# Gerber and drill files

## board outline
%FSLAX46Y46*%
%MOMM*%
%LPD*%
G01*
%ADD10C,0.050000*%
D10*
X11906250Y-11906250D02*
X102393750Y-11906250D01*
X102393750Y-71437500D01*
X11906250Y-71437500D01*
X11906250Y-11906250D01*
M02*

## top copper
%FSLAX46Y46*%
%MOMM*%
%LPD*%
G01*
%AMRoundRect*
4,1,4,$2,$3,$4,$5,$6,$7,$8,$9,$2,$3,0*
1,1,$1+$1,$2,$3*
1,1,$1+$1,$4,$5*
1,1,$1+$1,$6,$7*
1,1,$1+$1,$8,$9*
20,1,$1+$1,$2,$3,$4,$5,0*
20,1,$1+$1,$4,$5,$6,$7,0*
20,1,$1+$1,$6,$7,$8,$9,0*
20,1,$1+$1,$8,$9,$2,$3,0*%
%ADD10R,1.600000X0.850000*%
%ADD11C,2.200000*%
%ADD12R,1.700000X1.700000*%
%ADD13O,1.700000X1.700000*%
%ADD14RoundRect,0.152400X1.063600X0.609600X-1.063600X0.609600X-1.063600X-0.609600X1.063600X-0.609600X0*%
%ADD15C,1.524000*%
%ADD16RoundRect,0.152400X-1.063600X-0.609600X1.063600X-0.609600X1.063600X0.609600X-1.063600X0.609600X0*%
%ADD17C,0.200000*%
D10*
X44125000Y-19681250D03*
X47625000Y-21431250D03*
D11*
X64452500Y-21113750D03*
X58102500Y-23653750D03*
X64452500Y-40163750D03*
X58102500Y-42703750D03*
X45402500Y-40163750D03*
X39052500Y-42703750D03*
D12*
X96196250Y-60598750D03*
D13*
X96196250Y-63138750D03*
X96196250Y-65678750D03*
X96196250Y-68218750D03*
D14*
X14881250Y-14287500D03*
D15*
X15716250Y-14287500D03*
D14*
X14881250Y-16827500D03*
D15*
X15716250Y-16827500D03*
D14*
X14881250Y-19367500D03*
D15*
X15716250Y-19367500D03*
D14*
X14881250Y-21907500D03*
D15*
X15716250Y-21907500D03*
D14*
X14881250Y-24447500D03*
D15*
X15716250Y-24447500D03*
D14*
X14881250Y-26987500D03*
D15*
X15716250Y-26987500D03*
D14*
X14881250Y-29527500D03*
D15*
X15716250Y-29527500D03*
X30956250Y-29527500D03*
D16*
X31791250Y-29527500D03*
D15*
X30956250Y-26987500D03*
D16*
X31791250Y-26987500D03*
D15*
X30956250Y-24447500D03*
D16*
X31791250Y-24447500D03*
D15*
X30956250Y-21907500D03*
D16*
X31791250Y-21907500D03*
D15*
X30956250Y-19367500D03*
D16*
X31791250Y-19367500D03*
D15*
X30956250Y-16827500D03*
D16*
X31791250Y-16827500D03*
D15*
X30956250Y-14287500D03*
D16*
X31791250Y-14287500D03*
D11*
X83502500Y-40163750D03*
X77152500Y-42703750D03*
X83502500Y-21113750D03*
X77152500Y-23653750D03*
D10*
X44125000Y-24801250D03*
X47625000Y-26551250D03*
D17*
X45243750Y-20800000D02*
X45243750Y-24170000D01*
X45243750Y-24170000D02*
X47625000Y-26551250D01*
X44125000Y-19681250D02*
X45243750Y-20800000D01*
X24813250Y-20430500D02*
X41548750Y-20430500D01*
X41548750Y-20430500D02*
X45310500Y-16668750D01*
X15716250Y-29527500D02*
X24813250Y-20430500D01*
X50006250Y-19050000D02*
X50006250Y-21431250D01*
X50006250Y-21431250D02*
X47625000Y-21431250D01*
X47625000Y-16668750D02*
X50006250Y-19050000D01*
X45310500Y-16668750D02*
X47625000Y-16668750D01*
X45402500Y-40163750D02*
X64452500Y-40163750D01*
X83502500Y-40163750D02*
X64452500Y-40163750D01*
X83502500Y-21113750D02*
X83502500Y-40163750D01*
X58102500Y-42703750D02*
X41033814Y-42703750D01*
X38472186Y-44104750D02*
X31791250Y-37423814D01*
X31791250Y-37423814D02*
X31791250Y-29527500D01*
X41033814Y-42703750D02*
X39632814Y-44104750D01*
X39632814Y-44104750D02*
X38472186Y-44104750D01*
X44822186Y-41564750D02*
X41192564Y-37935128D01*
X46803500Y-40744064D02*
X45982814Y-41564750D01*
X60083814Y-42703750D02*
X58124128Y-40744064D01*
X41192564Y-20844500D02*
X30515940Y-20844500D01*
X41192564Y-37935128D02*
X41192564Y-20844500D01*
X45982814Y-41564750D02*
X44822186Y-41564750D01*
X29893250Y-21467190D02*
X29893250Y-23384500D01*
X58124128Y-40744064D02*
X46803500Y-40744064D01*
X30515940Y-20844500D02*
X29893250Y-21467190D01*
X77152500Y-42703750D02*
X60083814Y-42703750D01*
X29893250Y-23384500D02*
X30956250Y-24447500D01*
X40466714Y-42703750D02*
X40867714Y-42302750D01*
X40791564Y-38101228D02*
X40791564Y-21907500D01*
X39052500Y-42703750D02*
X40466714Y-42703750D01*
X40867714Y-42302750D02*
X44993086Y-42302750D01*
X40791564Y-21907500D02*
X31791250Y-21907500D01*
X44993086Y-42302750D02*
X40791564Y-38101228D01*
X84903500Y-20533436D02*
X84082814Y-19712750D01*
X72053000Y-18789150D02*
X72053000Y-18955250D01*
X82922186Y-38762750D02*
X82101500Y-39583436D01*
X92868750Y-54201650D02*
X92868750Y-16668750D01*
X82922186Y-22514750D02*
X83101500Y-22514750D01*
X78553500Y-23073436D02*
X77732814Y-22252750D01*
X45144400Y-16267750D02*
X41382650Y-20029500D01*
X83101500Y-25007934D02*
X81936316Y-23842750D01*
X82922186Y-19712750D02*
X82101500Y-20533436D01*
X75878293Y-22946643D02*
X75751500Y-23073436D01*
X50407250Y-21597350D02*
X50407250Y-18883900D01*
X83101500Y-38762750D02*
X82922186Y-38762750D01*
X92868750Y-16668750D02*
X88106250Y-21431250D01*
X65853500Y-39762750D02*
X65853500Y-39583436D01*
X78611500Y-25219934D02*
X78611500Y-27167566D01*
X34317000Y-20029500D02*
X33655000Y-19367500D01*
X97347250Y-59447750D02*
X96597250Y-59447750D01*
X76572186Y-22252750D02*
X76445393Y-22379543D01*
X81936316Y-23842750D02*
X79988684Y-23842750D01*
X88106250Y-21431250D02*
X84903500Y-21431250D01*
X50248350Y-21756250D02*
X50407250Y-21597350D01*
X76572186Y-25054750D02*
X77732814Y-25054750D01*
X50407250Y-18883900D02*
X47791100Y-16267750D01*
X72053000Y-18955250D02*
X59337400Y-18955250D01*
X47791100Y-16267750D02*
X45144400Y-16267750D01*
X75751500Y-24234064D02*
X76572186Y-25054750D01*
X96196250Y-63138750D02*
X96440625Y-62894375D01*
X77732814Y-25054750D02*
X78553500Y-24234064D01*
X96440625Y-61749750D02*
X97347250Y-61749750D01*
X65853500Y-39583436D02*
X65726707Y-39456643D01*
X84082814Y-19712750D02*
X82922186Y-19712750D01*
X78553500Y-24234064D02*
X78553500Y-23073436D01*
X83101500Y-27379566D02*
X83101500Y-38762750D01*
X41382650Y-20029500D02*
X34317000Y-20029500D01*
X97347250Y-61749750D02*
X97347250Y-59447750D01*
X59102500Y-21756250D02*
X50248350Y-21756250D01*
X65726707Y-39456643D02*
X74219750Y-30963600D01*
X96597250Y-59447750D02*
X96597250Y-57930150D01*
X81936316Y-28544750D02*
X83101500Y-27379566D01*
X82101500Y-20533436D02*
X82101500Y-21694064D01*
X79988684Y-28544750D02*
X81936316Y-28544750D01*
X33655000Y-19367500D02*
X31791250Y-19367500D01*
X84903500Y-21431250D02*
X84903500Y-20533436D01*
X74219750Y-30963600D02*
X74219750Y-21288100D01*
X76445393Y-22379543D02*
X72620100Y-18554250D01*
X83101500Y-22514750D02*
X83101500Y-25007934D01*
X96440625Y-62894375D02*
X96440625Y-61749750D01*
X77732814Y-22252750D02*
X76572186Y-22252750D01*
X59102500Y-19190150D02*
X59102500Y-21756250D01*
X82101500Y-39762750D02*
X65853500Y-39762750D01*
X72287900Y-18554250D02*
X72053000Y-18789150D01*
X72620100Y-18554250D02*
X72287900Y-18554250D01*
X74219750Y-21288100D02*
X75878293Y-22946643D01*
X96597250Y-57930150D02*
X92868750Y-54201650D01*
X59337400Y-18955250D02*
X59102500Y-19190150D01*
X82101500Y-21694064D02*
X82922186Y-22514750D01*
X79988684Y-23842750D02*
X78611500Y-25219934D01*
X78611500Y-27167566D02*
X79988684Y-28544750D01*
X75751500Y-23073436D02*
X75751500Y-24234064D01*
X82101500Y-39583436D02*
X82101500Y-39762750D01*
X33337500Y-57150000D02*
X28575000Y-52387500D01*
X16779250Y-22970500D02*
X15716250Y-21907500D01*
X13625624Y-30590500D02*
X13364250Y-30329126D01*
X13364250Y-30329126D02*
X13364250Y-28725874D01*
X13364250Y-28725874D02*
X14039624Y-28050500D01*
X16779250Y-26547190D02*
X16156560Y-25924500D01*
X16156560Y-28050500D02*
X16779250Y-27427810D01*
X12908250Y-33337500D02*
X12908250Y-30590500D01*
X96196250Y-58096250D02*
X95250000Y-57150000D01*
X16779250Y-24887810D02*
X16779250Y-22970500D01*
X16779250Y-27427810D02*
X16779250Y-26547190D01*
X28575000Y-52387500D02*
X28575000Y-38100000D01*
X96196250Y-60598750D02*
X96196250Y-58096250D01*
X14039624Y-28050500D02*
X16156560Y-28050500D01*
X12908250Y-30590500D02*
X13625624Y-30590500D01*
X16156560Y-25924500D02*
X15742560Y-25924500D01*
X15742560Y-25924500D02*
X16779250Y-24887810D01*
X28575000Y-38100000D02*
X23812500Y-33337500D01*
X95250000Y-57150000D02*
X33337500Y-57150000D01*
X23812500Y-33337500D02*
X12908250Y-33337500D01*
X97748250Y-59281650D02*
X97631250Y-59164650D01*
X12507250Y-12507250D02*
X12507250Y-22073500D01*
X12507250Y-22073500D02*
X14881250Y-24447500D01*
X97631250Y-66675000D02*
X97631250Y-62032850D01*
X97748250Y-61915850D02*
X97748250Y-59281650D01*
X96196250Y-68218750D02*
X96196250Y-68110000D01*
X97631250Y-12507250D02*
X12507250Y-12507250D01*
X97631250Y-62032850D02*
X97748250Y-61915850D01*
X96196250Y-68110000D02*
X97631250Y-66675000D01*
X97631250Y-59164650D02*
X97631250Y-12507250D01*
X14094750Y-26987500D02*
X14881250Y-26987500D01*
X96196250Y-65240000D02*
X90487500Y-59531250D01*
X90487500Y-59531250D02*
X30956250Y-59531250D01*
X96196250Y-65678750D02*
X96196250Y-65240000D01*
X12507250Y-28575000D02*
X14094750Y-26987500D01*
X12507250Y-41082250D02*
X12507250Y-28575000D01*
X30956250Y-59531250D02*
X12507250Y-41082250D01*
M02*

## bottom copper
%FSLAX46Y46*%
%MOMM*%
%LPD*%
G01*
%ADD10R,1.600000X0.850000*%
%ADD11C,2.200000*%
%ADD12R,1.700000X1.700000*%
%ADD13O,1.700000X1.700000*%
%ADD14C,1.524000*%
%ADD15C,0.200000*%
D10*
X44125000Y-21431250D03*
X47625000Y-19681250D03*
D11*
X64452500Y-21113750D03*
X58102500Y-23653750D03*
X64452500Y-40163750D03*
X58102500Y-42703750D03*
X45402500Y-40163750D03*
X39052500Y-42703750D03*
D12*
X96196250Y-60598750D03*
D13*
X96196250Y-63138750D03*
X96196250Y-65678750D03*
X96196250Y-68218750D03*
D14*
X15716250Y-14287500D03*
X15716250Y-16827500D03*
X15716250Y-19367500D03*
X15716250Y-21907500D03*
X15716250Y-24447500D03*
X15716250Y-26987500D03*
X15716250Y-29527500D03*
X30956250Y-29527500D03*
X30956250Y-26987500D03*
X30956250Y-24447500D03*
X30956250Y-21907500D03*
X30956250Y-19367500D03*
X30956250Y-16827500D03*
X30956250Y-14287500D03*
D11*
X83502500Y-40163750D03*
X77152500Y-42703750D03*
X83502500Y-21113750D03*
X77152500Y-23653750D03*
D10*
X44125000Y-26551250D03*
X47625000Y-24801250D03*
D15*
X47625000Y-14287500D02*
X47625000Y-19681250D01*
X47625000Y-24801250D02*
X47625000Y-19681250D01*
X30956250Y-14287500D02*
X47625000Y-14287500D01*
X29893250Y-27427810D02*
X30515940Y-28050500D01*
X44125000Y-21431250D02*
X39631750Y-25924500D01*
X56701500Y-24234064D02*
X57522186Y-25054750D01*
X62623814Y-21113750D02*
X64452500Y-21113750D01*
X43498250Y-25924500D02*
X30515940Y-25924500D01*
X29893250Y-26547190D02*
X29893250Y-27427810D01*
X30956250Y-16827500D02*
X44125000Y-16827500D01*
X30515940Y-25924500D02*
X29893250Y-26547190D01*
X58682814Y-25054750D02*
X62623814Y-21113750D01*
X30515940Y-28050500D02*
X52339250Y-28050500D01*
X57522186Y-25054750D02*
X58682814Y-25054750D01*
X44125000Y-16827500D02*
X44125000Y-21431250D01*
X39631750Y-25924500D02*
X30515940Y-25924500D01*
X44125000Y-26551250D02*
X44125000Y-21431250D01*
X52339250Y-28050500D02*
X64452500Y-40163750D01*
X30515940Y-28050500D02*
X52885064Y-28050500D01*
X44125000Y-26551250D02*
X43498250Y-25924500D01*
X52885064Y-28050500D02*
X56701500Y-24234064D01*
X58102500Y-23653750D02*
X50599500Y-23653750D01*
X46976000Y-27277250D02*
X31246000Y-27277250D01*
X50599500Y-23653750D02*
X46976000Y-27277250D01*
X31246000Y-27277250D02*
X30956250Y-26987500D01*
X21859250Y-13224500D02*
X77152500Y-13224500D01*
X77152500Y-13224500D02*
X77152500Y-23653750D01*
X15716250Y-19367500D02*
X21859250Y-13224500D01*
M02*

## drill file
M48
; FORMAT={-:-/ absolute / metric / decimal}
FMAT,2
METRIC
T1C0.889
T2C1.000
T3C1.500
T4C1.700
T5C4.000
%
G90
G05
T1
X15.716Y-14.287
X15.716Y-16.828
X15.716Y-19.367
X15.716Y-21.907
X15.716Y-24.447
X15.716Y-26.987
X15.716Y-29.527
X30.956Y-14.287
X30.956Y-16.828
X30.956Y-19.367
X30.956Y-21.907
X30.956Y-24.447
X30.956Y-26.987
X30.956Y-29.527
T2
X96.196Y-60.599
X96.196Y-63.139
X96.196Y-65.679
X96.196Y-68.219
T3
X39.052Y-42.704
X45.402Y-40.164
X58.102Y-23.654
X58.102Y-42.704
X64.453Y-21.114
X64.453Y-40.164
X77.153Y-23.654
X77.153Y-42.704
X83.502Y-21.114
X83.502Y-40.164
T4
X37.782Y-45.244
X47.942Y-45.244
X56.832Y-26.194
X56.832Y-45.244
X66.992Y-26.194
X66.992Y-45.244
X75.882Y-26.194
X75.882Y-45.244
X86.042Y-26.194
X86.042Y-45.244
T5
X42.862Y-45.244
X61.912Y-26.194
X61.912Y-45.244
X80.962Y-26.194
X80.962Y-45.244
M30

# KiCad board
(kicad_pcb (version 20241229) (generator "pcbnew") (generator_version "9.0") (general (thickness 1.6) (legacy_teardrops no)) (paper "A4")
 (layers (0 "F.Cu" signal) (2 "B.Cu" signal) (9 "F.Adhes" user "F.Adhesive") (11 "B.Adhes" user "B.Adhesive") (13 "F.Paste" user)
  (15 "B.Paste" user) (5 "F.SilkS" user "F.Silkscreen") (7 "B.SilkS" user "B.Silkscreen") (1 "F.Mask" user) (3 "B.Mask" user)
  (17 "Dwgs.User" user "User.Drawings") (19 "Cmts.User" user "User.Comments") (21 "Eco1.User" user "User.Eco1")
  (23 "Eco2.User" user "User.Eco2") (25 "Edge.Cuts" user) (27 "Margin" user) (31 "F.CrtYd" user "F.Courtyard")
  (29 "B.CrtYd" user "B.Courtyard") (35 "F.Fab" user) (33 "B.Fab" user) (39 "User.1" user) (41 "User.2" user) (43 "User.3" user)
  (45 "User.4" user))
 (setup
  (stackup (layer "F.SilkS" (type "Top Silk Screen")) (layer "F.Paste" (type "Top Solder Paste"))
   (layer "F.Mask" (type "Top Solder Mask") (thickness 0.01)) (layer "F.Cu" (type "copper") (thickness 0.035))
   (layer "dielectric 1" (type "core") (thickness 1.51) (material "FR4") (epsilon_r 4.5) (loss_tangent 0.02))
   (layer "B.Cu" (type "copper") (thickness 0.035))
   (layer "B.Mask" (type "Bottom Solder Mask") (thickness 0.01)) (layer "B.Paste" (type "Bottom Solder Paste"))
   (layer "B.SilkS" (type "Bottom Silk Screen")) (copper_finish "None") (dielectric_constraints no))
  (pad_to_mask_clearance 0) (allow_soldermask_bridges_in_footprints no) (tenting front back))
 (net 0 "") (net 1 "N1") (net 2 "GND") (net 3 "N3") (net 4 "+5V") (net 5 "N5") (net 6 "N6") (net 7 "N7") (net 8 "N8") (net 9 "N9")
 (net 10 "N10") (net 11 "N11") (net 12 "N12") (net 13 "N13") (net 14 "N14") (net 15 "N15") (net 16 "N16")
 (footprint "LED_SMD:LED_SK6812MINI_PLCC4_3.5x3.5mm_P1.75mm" (layer "F.Cu") (at 45.875 20.55625)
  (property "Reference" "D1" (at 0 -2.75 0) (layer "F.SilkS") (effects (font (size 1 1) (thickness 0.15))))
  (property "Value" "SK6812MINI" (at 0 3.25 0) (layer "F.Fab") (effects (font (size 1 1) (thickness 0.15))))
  (pad "1" smd rect (at -1.75 -0.875) (size 1.6 0.85) (layers "F.Cu" "F.Mask" "F.Paste") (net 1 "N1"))
  (pad "2" smd rect (at -1.75 0.875) (size 1.6 0.85) (layers "F.Mask" "B.Cu" "F.Paste") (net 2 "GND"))
  (pad "3" smd rect (at 1.75 0.875) (size 1.6 0.85) (layers "F.Cu" "F.Mask" "F.Paste") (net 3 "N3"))
  (pad "4" smd rect (at 1.75 -0.875) (size 1.6 0.85) (layers "F.Mask" "B.Cu" "F.Paste") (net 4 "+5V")))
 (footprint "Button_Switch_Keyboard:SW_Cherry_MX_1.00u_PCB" (layer "F.Cu") (at 64.4525 21.11375)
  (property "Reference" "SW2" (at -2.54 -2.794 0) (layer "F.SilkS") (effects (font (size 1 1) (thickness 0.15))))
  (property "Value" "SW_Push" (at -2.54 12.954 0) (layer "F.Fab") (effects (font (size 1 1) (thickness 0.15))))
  (pad "" np_thru_hole circle (at -7.62 5.08) (size 1.7 1.7) (drill 1.7) (layers "*.Cu" "*.Mask"))
  (pad "" np_thru_hole circle (at -2.54 5.08) (size 4 4) (drill 4) (layers "*.Cu" "*.Mask"))
  (pad "" np_thru_hole circle (at 2.54 5.08) (size 1.7 1.7) (drill 1.7) (layers "*.Cu" "*.Mask"))
  (pad "1" thru_hole circle (at 0 0) (size 2.2 2.2) (drill 1.5) (layers "*.Cu" "*.Mask") (remove_unused_layers no) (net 2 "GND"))
  (pad "2" thru_hole circle (at -6.35 2.54) (size 2.2 2.2) (drill 1.5) (layers "*.Cu" "*.Mask") (remove_unused_layers no) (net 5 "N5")))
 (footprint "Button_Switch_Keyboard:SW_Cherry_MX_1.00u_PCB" (layer "F.Cu") (at 64.4525 40.16375)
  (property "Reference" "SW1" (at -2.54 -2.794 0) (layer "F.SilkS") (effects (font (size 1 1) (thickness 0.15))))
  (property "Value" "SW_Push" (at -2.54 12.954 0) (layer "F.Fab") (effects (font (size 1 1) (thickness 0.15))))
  (pad "" np_thru_hole circle (at -7.62 5.08) (size 1.7 1.7) (drill 1.7) (layers "*.Cu" "*.Mask"))
  (pad "" np_thru_hole circle (at -2.54 5.08) (size 4 4) (drill 4) (layers "*.Cu" "*.Mask"))
  (pad "" np_thru_hole circle (at 2.54 5.08) (size 1.7 1.7) (drill 1.7) (layers "*.Cu" "*.Mask"))
  (pad "1" thru_hole circle (at 0 0) (size 2.2 2.2) (drill 1.5) (layers "*.Cu" "*.Mask") (remove_unused_layers no) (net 2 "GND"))
  (pad "2" thru_hole circle (at -6.35 2.54) (size 2.2 2.2) (drill 1.5) (layers "*.Cu" "*.Mask") (remove_unused_layers no) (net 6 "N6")))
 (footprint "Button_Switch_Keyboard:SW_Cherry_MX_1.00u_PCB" (layer "F.Cu") (at 45.4025 40.16375)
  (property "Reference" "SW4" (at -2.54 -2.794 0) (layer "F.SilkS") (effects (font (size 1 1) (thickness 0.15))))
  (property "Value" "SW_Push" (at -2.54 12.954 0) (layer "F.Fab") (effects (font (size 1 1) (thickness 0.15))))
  (pad "" np_thru_hole circle (at -7.62 5.08) (size 1.7 1.7) (drill 1.7) (layers "*.Cu" "*.Mask"))
  (pad "" np_thru_hole circle (at -2.54 5.08) (size 4 4) (drill 4) (layers "*.Cu" "*.Mask"))
  (pad "" np_thru_hole circle (at 2.54 5.08) (size 1.7 1.7) (drill 1.7) (layers "*.Cu" "*.Mask"))
  (pad "1" thru_hole circle (at 0 0) (size 2.2 2.2) (drill 1.5) (layers "*.Cu" "*.Mask") (remove_unused_layers no) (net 2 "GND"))
  (pad "2" thru_hole circle (at -6.35 2.54) (size 2.2 2.2) (drill 1.5) (layers "*.Cu" "*.Mask") (remove_unused_layers no) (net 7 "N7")))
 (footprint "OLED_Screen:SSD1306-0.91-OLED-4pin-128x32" (layer "F.Cu") (at 59.69625 58.40875)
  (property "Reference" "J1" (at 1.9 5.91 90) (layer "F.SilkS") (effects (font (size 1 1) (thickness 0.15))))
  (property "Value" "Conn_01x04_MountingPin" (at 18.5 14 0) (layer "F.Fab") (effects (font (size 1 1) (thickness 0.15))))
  (pad "1" thru_hole rect (at 36.5 2.19) (size 1.7 1.7) (drill 1) (layers "*.Cu" "*.Mask") (remove_unused_layers no) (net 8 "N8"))
  (pad "2" thru_hole oval (at 36.5 4.73) (size 1.7 1.7) (drill 1) (layers "*.Cu" "*.Mask") (remove_unused_layers no) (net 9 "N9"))
  (pad "3" thru_hole oval (at 36.5 7.27) (size 1.7 1.7) (drill 1) (layers "*.Cu" "*.Mask") (remove_unused_layers no) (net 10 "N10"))
  (pad "4" thru_hole oval (at 36.5 9.81) (size 1.7 1.7) (drill 1) (layers "*.Cu" "*.Mask") (remove_unused_layers no) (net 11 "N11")))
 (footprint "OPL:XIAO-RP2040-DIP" (layer "F.Cu") (at 23.33625 21.9075)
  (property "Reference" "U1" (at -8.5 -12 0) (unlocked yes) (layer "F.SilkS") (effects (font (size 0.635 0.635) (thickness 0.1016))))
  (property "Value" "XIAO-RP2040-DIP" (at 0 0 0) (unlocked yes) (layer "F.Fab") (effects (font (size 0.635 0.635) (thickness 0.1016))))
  (pad "1" smd roundrect (at -8.455 -7.62 180) (size 2.432 1.524) (layers "F.Cu" "F.Mask") (roundrect_rratio 0.1) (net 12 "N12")
   (thermal_bridge_angle 45))
  (pad "1" thru_hole circle (at -7.62 -7.62 180) (size 1.524 1.524) (drill 0.889) (layers "*.Cu" "*.Mask") (remove_unused_layers no)
   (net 12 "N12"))
  (pad "2" smd roundrect (at -8.455 -5.08 180) (size 2.432 1.524) (layers "F.Cu" "F.Mask") (roundrect_rratio 0.1) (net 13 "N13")
   (thermal_bridge_angle 45))
  (pad "2" thru_hole circle (at -7.62 -5.08 180) (size 1.524 1.524) (drill 0.889) (layers "*.Cu" "*.Mask") (remove_unused_layers no)
   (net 13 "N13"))
  (pad "3" smd roundrect (at -8.455 -2.54 180) (size 2.432 1.524) (layers "F.Cu" "F.Mask") (roundrect_rratio 0.1) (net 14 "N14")
   (thermal_bridge_angle 45))
  (pad "3" thru_hole circle (at -7.62 -2.54 180) (size 1.524 1.524) (drill 0.889) (layers "*.Cu" "*.Mask") (remove_unused_layers no)
   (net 14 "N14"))
  (pad "4" smd roundrect (at -8.455 0 180) (size 2.432 1.524) (layers "F.Cu" "F.Mask") (roundrect_rratio 0.1) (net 8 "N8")
   (thermal_bridge_angle 45))
  (pad "4" thru_hole circle (at -7.62 0 180) (size 1.524 1.524) (drill 0.889) (layers "*.Cu" "*.Mask") (remove_unused_layers no)
   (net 8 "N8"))
  (pad "5" smd roundrect (at -8.455 2.54 180) (size 2.432 1.524) (layers "F.Cu" "F.Mask") (roundrect_rratio 0.1) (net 11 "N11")
   (thermal_bridge_angle 45))
  (pad "5" thru_hole circle (at -7.62 2.54 180) (size 1.524 1.524) (drill 0.889) (layers "*.Cu" "*.Mask") (remove_unused_layers no)
   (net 11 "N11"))
  (pad "6" smd roundrect (at -8.455 5.08 180) (size 2.432 1.524) (layers "F.Cu" "F.Mask") (roundrect_rratio 0.1) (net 10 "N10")
   (thermal_bridge_angle 45))
  (pad "6" thru_hole circle (at -7.62 5.08 180) (size 1.524 1.524) (drill 0.889) (layers "*.Cu" "*.Mask") (remove_unused_layers no)
   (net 10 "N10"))
  (pad "7" smd roundrect (at -8.455 7.62 180) (size 2.432 1.524) (layers "F.Cu" "F.Mask") (roundrect_rratio 0.1) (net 3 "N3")
   (thermal_bridge_angle 45))
  (pad "7" thru_hole circle (at -7.62 7.62 180) (size 1.524 1.524) (drill 0.889) (layers "*.Cu" "*.Mask") (remove_unused_layers no)
   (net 3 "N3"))
  (pad "8" thru_hole circle (at 7.62 7.62) (size 1.524 1.524) (drill 0.889) (layers "*.Cu" "*.Mask") (remove_unused_layers no) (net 6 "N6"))
  (pad "8" smd roundrect (at 8.455 7.62) (size 2.432 1.524) (layers "F.Cu" "F.Mask") (roundrect_rratio 0.1) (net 6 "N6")
   (thermal_bridge_angle 45))
  (pad "9" thru_hole circle (at 7.62 5.08) (size 1.524 1.524) (drill 0.889) (layers "*.Cu" "*.Mask") (remove_unused_layers no) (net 5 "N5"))
  (pad "9" smd roundrect (at 8.455 5.08) (size 2.432 1.524) (layers "F.Cu" "F.Mask") (roundrect_rratio 0.1) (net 5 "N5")
   (thermal_bridge_angle 45))
  (pad "10" thru_hole circle (at 7.62 2.54) (size 1.524 1.524) (drill 0.889) (layers "*.Cu" "*.Mask") (remove_unused_layers no)
   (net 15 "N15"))
  (pad "10" smd roundrect (at 8.455 2.54) (size 2.432 1.524) (layers "F.Cu" "F.Mask") (roundrect_rratio 0.1) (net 15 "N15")
   (thermal_bridge_angle 45))
  (pad "11" thru_hole circle (at 7.62 0) (size 1.524 1.524) (drill 0.889) (layers "*.Cu" "*.Mask") (remove_unused_layers no) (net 7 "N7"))
  (pad "11" smd roundrect (at 8.455 0) (size 2.432 1.524) (layers "F.Cu" "F.Mask") (roundrect_rratio 0.1) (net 7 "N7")
   (thermal_bridge_angle 45))
  (pad "12" thru_hole circle (at 7.62 -2.54) (size 1.524 1.524) (drill 0.889) (layers "*.Cu" "*.Mask") (remove_unused_layers no)
   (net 9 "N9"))
  (pad "12" smd roundrect (at 8.455 -2.54) (size 2.432 1.524) (layers "F.Cu" "F.Mask") (roundrect_rratio 0.1) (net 9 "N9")
   (thermal_bridge_angle 45))
  (pad "13" thru_hole circle (at 7.62 -5.08) (size 1.524 1.524) (drill 0.889) (layers "*.Cu" "*.Mask") (remove_unused_layers no)
   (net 2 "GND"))
  (pad "13" smd roundrect (at 8.455 -5.08) (size 2.432 1.524) (layers "F.Cu" "F.Mask") (roundrect_rratio 0.1) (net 2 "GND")
   (thermal_bridge_angle 45))
  (pad "14" thru_hole circle (at 7.62 -7.62) (size 1.524 1.524) (drill 0.889) (layers "*.Cu" "*.Mask") (remove_unused_layers no)
   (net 4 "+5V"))
  (pad "14" smd roundrect (at 8.455 -7.62) (size 2.432 1.524) (layers "F.Cu" "F.Mask") (roundrect_rratio 0.1) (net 4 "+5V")
   (thermal_bridge_angle 45)))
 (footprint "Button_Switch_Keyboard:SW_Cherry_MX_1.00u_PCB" (layer "F.Cu") (at 83.5025 40.16375)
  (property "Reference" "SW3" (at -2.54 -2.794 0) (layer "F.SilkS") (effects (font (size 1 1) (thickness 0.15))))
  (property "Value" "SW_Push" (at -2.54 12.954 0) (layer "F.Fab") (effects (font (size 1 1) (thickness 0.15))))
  (pad "" np_thru_hole circle (at -7.62 5.08) (size 1.7 1.7) (drill 1.7) (layers "*.Cu" "*.Mask"))
  (pad "" np_thru_hole circle (at -2.54 5.08) (size 4 4) (drill 4) (layers "*.Cu" "*.Mask"))
  (pad "" np_thru_hole circle (at 2.54 5.08) (size 1.7 1.7) (drill 1.7) (layers "*.Cu" "*.Mask"))
  (pad "1" thru_hole circle (at 0 0) (size 2.2 2.2) (drill 1.5) (layers "*.Cu" "*.Mask") (remove_unused_layers no) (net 2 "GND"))
  (pad "2" thru_hole circle (at -6.35 2.54) (size 2.2 2.2) (drill 1.5) (layers "*.Cu" "*.Mask") (remove_unused_layers no) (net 15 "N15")))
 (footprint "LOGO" (layer "F.Cu") (at 21.43125 61.9125)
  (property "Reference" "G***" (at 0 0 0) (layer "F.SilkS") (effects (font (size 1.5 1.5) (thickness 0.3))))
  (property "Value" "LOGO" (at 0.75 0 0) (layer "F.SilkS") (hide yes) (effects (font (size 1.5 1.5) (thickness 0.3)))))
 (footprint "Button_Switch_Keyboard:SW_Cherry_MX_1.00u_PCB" (layer "F.Cu") (at 83.5025 21.11375)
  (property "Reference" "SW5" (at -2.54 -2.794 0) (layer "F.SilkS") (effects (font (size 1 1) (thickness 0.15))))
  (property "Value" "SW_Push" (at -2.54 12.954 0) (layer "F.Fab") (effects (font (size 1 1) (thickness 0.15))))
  (pad "" np_thru_hole circle (at -7.62 5.08) (size 1.7 1.7) (drill 1.7) (layers "*.Cu" "*.Mask"))
  (pad "" np_thru_hole circle (at -2.54 5.08) (size 4 4) (drill 4) (layers "*.Cu" "*.Mask"))
  (pad "" np_thru_hole circle (at 2.54 5.08) (size 1.7 1.7) (drill 1.7) (layers "*.Cu" "*.Mask"))
  (pad "1" thru_hole circle (at 0 0) (size 2.2 2.2) (drill 1.5) (layers "*.Cu" "*.Mask") (remove_unused_layers no) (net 2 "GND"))
  (pad "2" thru_hole circle (at -6.35 2.54) (size 2.2 2.2) (drill 1.5) (layers "*.Cu" "*.Mask") (remove_unused_layers no) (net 14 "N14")))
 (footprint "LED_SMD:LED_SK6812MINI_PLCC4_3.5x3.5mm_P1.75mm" (layer "F.Cu") (at 45.875 25.67625)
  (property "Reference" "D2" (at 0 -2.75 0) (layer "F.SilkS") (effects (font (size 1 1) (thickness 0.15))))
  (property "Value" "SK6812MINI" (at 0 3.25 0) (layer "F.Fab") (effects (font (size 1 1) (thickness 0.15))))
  (pad "1" smd rect (at -1.75 -0.875) (size 1.6 0.85) (layers "F.Cu" "F.Mask" "F.Paste") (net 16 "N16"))
  (pad "2" smd rect (at -1.75 0.875) (size 1.6 0.85) (layers "F.Mask" "B.Cu" "F.Paste") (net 2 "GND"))
  (pad "3" smd rect (at 1.75 0.875) (size 1.6 0.85) (layers "F.Cu" "F.Mask" "F.Paste") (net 1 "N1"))
  (pad "4" smd rect (at 1.75 -0.875) (size 1.6 0.85) (layers "F.Mask" "B.Cu" "F.Paste") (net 4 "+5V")))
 (gr_rect (start 11.90625 11.90625) (end 102.39375 71.4375) (stroke (width 0.05) (type default)) (fill no) (layer "Edge.Cuts"))
 (segment (start 45.24375 20.8) (end 45.24375 24.17) (width 0.2) (layer "F.Cu") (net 1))
 (segment (start 45.24375 24.17) (end 47.625 26.55125) (width 0.2) (layer "F.Cu") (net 1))
 (segment (start 44.125 19.68125) (end 45.24375 20.8) (width 0.2) (layer "F.Cu") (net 1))
 (segment (start 47.625 14.2875) (end 47.625 19.68125) (width 0.2) (layer "B.Cu") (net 4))
 (segment (start 47.625 24.80125) (end 47.625 19.68125) (width 0.2) (layer "B.Cu") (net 4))
 (segment (start 30.95625 14.2875) (end 47.625 14.2875) (width 0.2) (layer "B.Cu") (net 4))
 (segment (start 24.81325 20.4305) (end 41.54875 20.4305) (width 0.2) (layer "F.Cu") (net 3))
 (segment (start 41.54875 20.4305) (end 45.3105 16.66875) (width 0.2) (layer "F.Cu") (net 3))
 (segment (start 15.71625 29.5275) (end 24.81325 20.4305) (width 0.2) (layer "F.Cu") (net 3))
 (segment (start 50.00625 19.05) (end 50.00625 21.43125) (width 0.2) (layer "F.Cu") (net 3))
 (segment (start 50.00625 21.43125) (end 47.625 21.43125) (width 0.2) (layer "F.Cu") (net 3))
 (segment (start 47.625 16.66875) (end 50.00625 19.05) (width 0.2) (layer "F.Cu") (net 3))
 (segment (start 45.3105 16.66875) (end 47.625 16.66875) (width 0.2) (layer "F.Cu") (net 3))
 (segment (start 45.4025 40.16375) (end 64.4525 40.16375) (width 0.2) (layer "F.Cu") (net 2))
 (segment (start 83.5025 40.16375) (end 64.4525 40.16375) (width 0.2) (layer "F.Cu") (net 2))
 (segment (start 83.5025 21.11375) (end 83.5025 40.16375) (width 0.2) (layer "F.Cu") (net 2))
 (segment (start 29.89325 27.42781) (end 30.51594 28.0505) (width 0.2) (layer "B.Cu") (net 2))
 (segment (start 44.125 21.43125) (end 39.63175 25.9245) (width 0.2) (layer "B.Cu") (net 2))
 (segment (start 56.7015 24.234064) (end 57.522186 25.05475) (width 0.2) (layer "B.Cu") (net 2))
 (segment (start 62.623814 21.11375) (end 64.4525 21.11375) (width 0.2) (layer "B.Cu") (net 2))
 (segment (start 43.49825 25.9245) (end 30.51594 25.9245) (width 0.2) (layer "B.Cu") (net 2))
 (segment (start 29.89325 26.54719) (end 29.89325 27.42781) (width 0.2) (layer "B.Cu") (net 2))
 (segment (start 30.95625 16.8275) (end 44.125 16.8275) (width 0.2) (layer "B.Cu") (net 2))
 (segment (start 30.51594 25.9245) (end 29.89325 26.54719) (width 0.2) (layer "B.Cu") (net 2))
 (segment (start 58.682814 25.05475) (end 62.623814 21.11375) (width 0.2) (layer "B.Cu") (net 2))
 (segment (start 30.51594 28.0505) (end 52.33925 28.0505) (width 0.2) (layer "B.Cu") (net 2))
 (segment (start 57.522186 25.05475) (end 58.682814 25.05475) (width 0.2) (layer "B.Cu") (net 2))
 (segment (start 44.125 16.8275) (end 44.125 21.43125) (width 0.2) (layer "B.Cu") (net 2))
 (segment (start 39.63175 25.9245) (end 30.51594 25.9245) (width 0.2) (layer "B.Cu") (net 2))
 (segment (start 44.125 26.55125) (end 44.125 21.43125) (width 0.2) (layer "B.Cu") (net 2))
 (segment (start 52.33925 28.0505) (end 64.4525 40.16375) (width 0.2) (layer "B.Cu") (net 2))
 (segment (start 30.51594 28.0505) (end 52.885064 28.0505) (width 0.2) (layer "B.Cu") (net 2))
 (segment (start 44.125 26.55125) (end 43.49825 25.9245) (width 0.2) (layer "B.Cu") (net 2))
 (segment (start 52.885064 28.0505) (end 56.7015 24.234064) (width 0.2) (layer "B.Cu") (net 2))
 (segment (start 58.1025 42.70375) (end 41.033814 42.70375) (width 0.2) (layer "F.Cu") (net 6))
 (segment (start 38.472186 44.10475) (end 31.79125 37.423814) (width 0.2) (layer "F.Cu") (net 6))
 (segment (start 31.79125 37.423814) (end 31.79125 29.5275) (width 0.2) (layer "F.Cu") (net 6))
 (segment (start 41.033814 42.70375) (end 39.632814 44.10475) (width 0.2) (layer "F.Cu") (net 6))
 (segment (start 39.632814 44.10475) (end 38.472186 44.10475) (width 0.2) (layer "F.Cu") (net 6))
 (segment (start 58.1025 23.65375) (end 50.5995 23.65375) (width 0.2) (layer "B.Cu") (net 5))
 (segment (start 46.976 27.27725) (end 31.246 27.27725) (width 0.2) (layer "B.Cu") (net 5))
 (segment (start 50.5995 23.65375) (end 46.976 27.27725) (width 0.2) (layer "B.Cu") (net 5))
 (segment (start 31.246 27.27725) (end 30.95625 26.9875) (width 0.2) (layer "B.Cu") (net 5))
 (segment (start 44.822186 41.56475) (end 41.192564 37.935128) (width 0.2) (layer "F.Cu") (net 15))
 (segment (start 46.8035 40.744064) (end 45.982814 41.56475) (width 0.2) (layer "F.Cu") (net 15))
 (segment (start 60.083814 42.70375) (end 58.124128 40.744064) (width 0.2) (layer "F.Cu") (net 15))
 (segment (start 41.192564 20.8445) (end 30.51594 20.8445) (width 0.2) (layer "F.Cu") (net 15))
 (segment (start 41.192564 37.935128) (end 41.192564 20.8445) (width 0.2) (layer "F.Cu") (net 15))
 (segment (start 45.982814 41.56475) (end 44.822186 41.56475) (width 0.2) (layer "F.Cu") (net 15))
 (segment (start 29.89325 21.46719) (end 29.89325 23.3845) (width 0.2) (layer "F.Cu") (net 15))
 (segment (start 58.124128 40.744064) (end 46.8035 40.744064) (width 0.2) (layer "F.Cu") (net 15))
 (segment (start 30.51594 20.8445) (end 29.89325 21.46719) (width 0.2) (layer "F.Cu") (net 15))
 (segment (start 77.1525 42.70375) (end 60.083814 42.70375) (width 0.2) (layer "F.Cu") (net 15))
 (segment (start 29.89325 23.3845) (end 30.95625 24.4475) (width 0.2) (layer "F.Cu") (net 15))
 (segment (start 40.466714 42.70375) (end 40.867714 42.30275) (width 0.2) (layer "F.Cu") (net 7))
 (segment (start 40.791564 38.101228) (end 40.791564 21.9075) (width 0.2) (layer "F.Cu") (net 7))
 (segment (start 39.0525 42.70375) (end 40.466714 42.70375) (width 0.2) (layer "F.Cu") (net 7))
 (segment (start 40.867714 42.30275) (end 44.993086 42.30275) (width 0.2) (layer "F.Cu") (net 7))
 (segment (start 40.791564 21.9075) (end 31.79125 21.9075) (width 0.2) (layer "F.Cu") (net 7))
 (segment (start 44.993086 42.30275) (end 40.791564 38.101228) (width 0.2) (layer "F.Cu") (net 7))
 (segment (start 84.9035 20.533436) (end 84.082814 19.71275) (width 0.2) (layer "F.Cu") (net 9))
 (segment (start 72.053 18.78915) (end 72.053 18.95525) (width 0.2) (layer "F.Cu") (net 9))
 (segment (start 82.922186 38.76275) (end 82.1015 39.583436) (width 0.2) (layer "F.Cu") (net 9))
 (segment (start 92.86875 54.20165) (end 92.86875 16.66875) (width 0.2) (layer "F.Cu") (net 9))
 (segment (start 82.922186 22.51475) (end 83.1015 22.51475) (width 0.2) (layer "F.Cu") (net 9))
 (segment (start 78.5535 23.073436) (end 77.732814 22.25275) (width 0.2) (layer "F.Cu") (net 9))
 (segment (start 45.1444 16.26775) (end 41.38265 20.0295) (width 0.2) (layer "F.Cu") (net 9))
 (segment (start 83.1015 25.007934) (end 81.936316 23.84275) (width 0.2) (layer "F.Cu") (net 9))
 (segment (start 82.922186 19.71275) (end 82.1015 20.533436) (width 0.2) (layer "F.Cu") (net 9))
 (segment (start 75.878293 22.946643) (end 75.7515 23.073436) (width 0.2) (layer "F.Cu") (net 9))
 (segment (start 50.40725 21.59735) (end 50.40725 18.8839) (width 0.2) (layer "F.Cu") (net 9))
 (segment (start 83.1015 38.76275) (end 82.922186 38.76275) (width 0.2) (layer "F.Cu") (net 9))
 (segment (start 92.86875 16.66875) (end 88.10625 21.43125) (width 0.2) (layer "F.Cu") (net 9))
 (segment (start 65.8535 39.76275) (end 65.8535 39.583436) (width 0.2) (layer "F.Cu") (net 9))
 (segment (start 78.6115 25.219934) (end 78.6115 27.167566) (width 0.2) (layer "F.Cu") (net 9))
 (segment (start 34.317 20.0295) (end 33.655 19.3675) (width 0.2) (layer "F.Cu") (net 9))
 (segment (start 97.34725 59.44775) (end 96.59725 59.44775) (width 0.2) (layer "F.Cu") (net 9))
 (segment (start 76.572186 22.25275) (end 76.445393 22.379543) (width 0.2) (layer "F.Cu") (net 9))
 (segment (start 81.936316 23.84275) (end 79.988684 23.84275) (width 0.2) (layer "F.Cu") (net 9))
 (segment (start 88.10625 21.43125) (end 84.9035 21.43125) (width 0.2) (layer "F.Cu") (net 9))
 (segment (start 50.24835 21.75625) (end 50.40725 21.59735) (width 0.2) (layer "F.Cu") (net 9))
 (segment (start 76.572186 25.05475) (end 77.732814 25.05475) (width 0.2) (layer "F.Cu") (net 9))
 (segment (start 50.40725 18.8839) (end 47.7911 16.26775) (width 0.2) (layer "F.Cu") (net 9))
 (segment (start 72.053 18.95525) (end 59.3374 18.95525) (width 0.2) (layer "F.Cu") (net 9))
 (segment (start 47.7911 16.26775) (end 45.1444 16.26775) (width 0.2) (layer "F.Cu") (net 9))
 (segment (start 75.7515 24.234064) (end 76.572186 25.05475) (width 0.2) (layer "F.Cu") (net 9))
 (segment (start 96.19625 63.13875) (end 96.440625 62.894375) (width 0.2) (layer "F.Cu") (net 9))
 (segment (start 77.732814 25.05475) (end 78.5535 24.234064) (width 0.2) (layer "F.Cu") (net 9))
 (segment (start 96.440625 61.74975) (end 97.34725 61.74975) (width 0.2) (layer "F.Cu") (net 9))
 (segment (start 65.8535 39.583436) (end 65.726707 39.456643) (width 0.2) (layer "F.Cu") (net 9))
 (segment (start 84.082814 19.71275) (end 82.922186 19.71275) (width 0.2) (layer "F.Cu") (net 9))
 (segment (start 78.5535 24.234064) (end 78.5535 23.073436) (width 0.2) (layer "F.Cu") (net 9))
 (segment (start 83.1015 27.379566) (end 83.1015 38.76275) (width 0.2) (layer "F.Cu") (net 9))
 (segment (start 41.38265 20.0295) (end 34.317 20.0295) (width 0.2) (layer "F.Cu") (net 9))
 (segment (start 97.34725 61.74975) (end 97.34725 59.44775) (width 0.2) (layer "F.Cu") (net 9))
 (segment (start 59.1025 21.75625) (end 50.24835 21.75625) (width 0.2) (layer "F.Cu") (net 9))
 (segment (start 65.726707 39.456643) (end 74.21975 30.9636) (width 0.2) (layer "F.Cu") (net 9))
 (segment (start 96.59725 59.44775) (end 96.59725 57.93015) (width 0.2) (layer "F.Cu") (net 9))
 (segment (start 81.936316 28.54475) (end 83.1015 27.379566) (width 0.2) (layer "F.Cu") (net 9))
 (segment (start 82.1015 20.533436) (end 82.1015 21.694064) (width 0.2) (layer "F.Cu") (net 9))
 (segment (start 79.988684 28.54475) (end 81.936316 28.54475) (width 0.2) (layer "F.Cu") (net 9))
 (segment (start 33.655 19.3675) (end 31.79125 19.3675) (width 0.2) (layer "F.Cu") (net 9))
 (segment (start 84.9035 21.43125) (end 84.9035 20.533436) (width 0.2) (layer "F.Cu") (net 9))
 (segment (start 74.21975 30.9636) (end 74.21975 21.2881) (width 0.2) (layer "F.Cu") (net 9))
 (segment (start 76.445393 22.379543) (end 72.6201 18.55425) (width 0.2) (layer "F.Cu") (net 9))
 (segment (start 83.1015 22.51475) (end 83.1015 25.007934) (width 0.2) (layer "F.Cu") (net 9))
 (segment (start 96.440625 62.894375) (end 96.440625 61.74975) (width 0.2) (layer "F.Cu") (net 9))
 (segment (start 77.732814 22.25275) (end 76.572186 22.25275) (width 0.2) (layer "F.Cu") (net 9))
 (segment (start 59.1025 19.19015) (end 59.1025 21.75625) (width 0.2) (layer "F.Cu") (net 9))
 (segment (start 82.1015 39.76275) (end 65.8535 39.76275) (width 0.2) (layer "F.Cu") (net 9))
 (segment (start 72.2879 18.55425) (end 72.053 18.78915) (width 0.2) (layer "F.Cu") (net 9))
 (segment (start 72.6201 18.55425) (end 72.2879 18.55425) (width 0.2) (layer "F.Cu") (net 9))
 (segment (start 74.21975 21.2881) (end 75.878293 22.946643) (width 0.2) (layer "F.Cu") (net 9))
 (segment (start 96.59725 57.93015) (end 92.86875 54.20165) (width 0.2) (layer "F.Cu") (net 9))
 (segment (start 59.3374 18.95525) (end 59.1025 19.19015) (width 0.2) (layer "F.Cu") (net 9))
 (segment (start 82.1015 21.694064) (end 82.922186 22.51475) (width 0.2) (layer "F.Cu") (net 9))
 (segment (start 79.988684 23.84275) (end 78.6115 25.219934) (width 0.2) (layer "F.Cu") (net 9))
 (segment (start 78.6115 27.167566) (end 79.988684 28.54475) (width 0.2) (layer "F.Cu") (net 9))
 (segment (start 75.7515 23.073436) (end 75.7515 24.234064) (width 0.2) (layer "F.Cu") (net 9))
 (segment (start 82.1015 39.583436) (end 82.1015 39.76275) (width 0.2) (layer "F.Cu") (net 9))
 (segment (start 33.3375 57.15) (end 28.575 52.3875) (width 0.2) (layer "F.Cu") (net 8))
 (segment (start 16.77925 22.9705) (end 15.71625 21.9075) (width 0.2) (layer "F.Cu") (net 8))
 (segment (start 13.625624 30.5905) (end 13.36425 30.329126) (width 0.2) (layer "F.Cu") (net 8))
 (segment (start 13.36425 30.329126) (end 13.36425 28.725874) (width 0.2) (layer "F.Cu") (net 8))
 (segment (start 13.36425 28.725874) (end 14.039624 28.0505) (width 0.2) (layer "F.Cu") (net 8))
 (segment (start 16.77925 26.54719) (end 16.15656 25.9245) (width 0.2) (layer "F.Cu") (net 8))
 (segment (start 16.15656 28.0505) (end 16.77925 27.42781) (width 0.2) (layer "F.Cu") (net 8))
 (segment (start 12.90825 33.3375) (end 12.90825 30.5905) (width 0.2) (layer "F.Cu") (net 8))
 (segment (start 96.19625 58.09625) (end 95.25 57.15) (width 0.2) (layer "F.Cu") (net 8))
 (segment (start 16.77925 24.88781) (end 16.77925 22.9705) (width 0.2) (layer "F.Cu") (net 8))
 (segment (start 16.77925 27.42781) (end 16.77925 26.54719) (width 0.2) (layer "F.Cu") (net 8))
 (segment (start 28.575 52.3875) (end 28.575 38.1) (width 0.2) (layer "F.Cu") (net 8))
 (segment (start 96.19625 60.59875) (end 96.19625 58.09625) (width 0.2) (layer "F.Cu") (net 8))
 (segment (start 14.039624 28.0505) (end 16.15656 28.0505) (width 0.2) (layer "F.Cu") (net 8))
 (segment (start 12.90825 30.5905) (end 13.625624 30.5905) (width 0.2) (layer "F.Cu") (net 8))
 (segment (start 16.15656 25.9245) (end 15.74256 25.9245) (width 0.2) (layer "F.Cu") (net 8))
 (segment (start 15.74256 25.9245) (end 16.77925 24.88781) (width 0.2) (layer "F.Cu") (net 8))
 (segment (start 28.575 38.1) (end 23.8125 33.3375) (width 0.2) (layer "F.Cu") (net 8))
 (segment (start 95.25 57.15) (end 33.3375 57.15) (width 0.2) (layer "F.Cu") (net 8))
 (segment (start 23.8125 33.3375) (end 12.90825 33.3375) (width 0.2) (layer "F.Cu") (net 8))
 (segment (start 97.74825 59.28165) (end 97.63125 59.16465) (width 0.2) (layer "F.Cu") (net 11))
 (segment (start 12.50725 12.50725) (end 12.50725 22.0735) (width 0.2) (layer "F.Cu") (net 11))
 (segment (start 12.50725 22.0735) (end 14.88125 24.4475) (width 0.2) (layer "F.Cu") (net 11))
 (segment (start 97.63125 66.675) (end 97.63125 62.03285) (width 0.2) (layer "F.Cu") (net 11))
 (segment (start 97.74825 61.91585) (end 97.74825 59.28165) (width 0.2) (layer "F.Cu") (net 11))
 (segment (start 96.19625 68.21875) (end 96.19625 68.11) (width 0.2) (layer "F.Cu") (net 11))
 (segment (start 97.63125 12.50725) (end 12.50725 12.50725) (width 0.2) (layer "F.Cu") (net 11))
 (segment (start 97.63125 62.03285) (end 97.74825 61.91585) (width 0.2) (layer "F.Cu") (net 11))
 (segment (start 96.19625 68.11) (end 97.63125 66.675) (width 0.2) (layer "F.Cu") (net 11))
 (segment (start 97.63125 59.16465) (end 97.63125 12.50725) (width 0.2) (layer "F.Cu") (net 11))
 (segment (start 14.09475 26.9875) (end 14.88125 26.9875) (width 0.2) (layer "F.Cu") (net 10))
 (segment (start 96.19625 65.24) (end 90.4875 59.53125) (width 0.2) (layer "F.Cu") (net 10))
 (segment (start 90.4875 59.53125) (end 30.95625 59.53125) (width 0.2) (layer "F.Cu") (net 10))
 (segment (start 96.19625 65.67875) (end 96.19625 65.24) (width 0.2) (layer "F.Cu") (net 10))
 (segment (start 12.50725 28.575) (end 14.09475 26.9875) (width 0.2) (layer "F.Cu") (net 10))
 (segment (start 12.50725 41.08225) (end 12.50725 28.575) (width 0.2) (layer "F.Cu") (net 10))
 (segment (start 30.95625 59.53125) (end 12.50725 41.08225) (width 0.2) (layer "F.Cu") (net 10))
 (segment (start 21.85925 13.2245) (end 77.1525 13.2245) (width 0.2) (layer "B.Cu") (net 14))
 (segment (start 77.1525 13.2245) (end 77.1525 23.65375) (width 0.2) (layer "B.Cu") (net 14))
 (segment (start 15.71625 19.3675) (end 21.85925 13.2245) (width 0.2) (layer "B.Cu") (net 14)))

